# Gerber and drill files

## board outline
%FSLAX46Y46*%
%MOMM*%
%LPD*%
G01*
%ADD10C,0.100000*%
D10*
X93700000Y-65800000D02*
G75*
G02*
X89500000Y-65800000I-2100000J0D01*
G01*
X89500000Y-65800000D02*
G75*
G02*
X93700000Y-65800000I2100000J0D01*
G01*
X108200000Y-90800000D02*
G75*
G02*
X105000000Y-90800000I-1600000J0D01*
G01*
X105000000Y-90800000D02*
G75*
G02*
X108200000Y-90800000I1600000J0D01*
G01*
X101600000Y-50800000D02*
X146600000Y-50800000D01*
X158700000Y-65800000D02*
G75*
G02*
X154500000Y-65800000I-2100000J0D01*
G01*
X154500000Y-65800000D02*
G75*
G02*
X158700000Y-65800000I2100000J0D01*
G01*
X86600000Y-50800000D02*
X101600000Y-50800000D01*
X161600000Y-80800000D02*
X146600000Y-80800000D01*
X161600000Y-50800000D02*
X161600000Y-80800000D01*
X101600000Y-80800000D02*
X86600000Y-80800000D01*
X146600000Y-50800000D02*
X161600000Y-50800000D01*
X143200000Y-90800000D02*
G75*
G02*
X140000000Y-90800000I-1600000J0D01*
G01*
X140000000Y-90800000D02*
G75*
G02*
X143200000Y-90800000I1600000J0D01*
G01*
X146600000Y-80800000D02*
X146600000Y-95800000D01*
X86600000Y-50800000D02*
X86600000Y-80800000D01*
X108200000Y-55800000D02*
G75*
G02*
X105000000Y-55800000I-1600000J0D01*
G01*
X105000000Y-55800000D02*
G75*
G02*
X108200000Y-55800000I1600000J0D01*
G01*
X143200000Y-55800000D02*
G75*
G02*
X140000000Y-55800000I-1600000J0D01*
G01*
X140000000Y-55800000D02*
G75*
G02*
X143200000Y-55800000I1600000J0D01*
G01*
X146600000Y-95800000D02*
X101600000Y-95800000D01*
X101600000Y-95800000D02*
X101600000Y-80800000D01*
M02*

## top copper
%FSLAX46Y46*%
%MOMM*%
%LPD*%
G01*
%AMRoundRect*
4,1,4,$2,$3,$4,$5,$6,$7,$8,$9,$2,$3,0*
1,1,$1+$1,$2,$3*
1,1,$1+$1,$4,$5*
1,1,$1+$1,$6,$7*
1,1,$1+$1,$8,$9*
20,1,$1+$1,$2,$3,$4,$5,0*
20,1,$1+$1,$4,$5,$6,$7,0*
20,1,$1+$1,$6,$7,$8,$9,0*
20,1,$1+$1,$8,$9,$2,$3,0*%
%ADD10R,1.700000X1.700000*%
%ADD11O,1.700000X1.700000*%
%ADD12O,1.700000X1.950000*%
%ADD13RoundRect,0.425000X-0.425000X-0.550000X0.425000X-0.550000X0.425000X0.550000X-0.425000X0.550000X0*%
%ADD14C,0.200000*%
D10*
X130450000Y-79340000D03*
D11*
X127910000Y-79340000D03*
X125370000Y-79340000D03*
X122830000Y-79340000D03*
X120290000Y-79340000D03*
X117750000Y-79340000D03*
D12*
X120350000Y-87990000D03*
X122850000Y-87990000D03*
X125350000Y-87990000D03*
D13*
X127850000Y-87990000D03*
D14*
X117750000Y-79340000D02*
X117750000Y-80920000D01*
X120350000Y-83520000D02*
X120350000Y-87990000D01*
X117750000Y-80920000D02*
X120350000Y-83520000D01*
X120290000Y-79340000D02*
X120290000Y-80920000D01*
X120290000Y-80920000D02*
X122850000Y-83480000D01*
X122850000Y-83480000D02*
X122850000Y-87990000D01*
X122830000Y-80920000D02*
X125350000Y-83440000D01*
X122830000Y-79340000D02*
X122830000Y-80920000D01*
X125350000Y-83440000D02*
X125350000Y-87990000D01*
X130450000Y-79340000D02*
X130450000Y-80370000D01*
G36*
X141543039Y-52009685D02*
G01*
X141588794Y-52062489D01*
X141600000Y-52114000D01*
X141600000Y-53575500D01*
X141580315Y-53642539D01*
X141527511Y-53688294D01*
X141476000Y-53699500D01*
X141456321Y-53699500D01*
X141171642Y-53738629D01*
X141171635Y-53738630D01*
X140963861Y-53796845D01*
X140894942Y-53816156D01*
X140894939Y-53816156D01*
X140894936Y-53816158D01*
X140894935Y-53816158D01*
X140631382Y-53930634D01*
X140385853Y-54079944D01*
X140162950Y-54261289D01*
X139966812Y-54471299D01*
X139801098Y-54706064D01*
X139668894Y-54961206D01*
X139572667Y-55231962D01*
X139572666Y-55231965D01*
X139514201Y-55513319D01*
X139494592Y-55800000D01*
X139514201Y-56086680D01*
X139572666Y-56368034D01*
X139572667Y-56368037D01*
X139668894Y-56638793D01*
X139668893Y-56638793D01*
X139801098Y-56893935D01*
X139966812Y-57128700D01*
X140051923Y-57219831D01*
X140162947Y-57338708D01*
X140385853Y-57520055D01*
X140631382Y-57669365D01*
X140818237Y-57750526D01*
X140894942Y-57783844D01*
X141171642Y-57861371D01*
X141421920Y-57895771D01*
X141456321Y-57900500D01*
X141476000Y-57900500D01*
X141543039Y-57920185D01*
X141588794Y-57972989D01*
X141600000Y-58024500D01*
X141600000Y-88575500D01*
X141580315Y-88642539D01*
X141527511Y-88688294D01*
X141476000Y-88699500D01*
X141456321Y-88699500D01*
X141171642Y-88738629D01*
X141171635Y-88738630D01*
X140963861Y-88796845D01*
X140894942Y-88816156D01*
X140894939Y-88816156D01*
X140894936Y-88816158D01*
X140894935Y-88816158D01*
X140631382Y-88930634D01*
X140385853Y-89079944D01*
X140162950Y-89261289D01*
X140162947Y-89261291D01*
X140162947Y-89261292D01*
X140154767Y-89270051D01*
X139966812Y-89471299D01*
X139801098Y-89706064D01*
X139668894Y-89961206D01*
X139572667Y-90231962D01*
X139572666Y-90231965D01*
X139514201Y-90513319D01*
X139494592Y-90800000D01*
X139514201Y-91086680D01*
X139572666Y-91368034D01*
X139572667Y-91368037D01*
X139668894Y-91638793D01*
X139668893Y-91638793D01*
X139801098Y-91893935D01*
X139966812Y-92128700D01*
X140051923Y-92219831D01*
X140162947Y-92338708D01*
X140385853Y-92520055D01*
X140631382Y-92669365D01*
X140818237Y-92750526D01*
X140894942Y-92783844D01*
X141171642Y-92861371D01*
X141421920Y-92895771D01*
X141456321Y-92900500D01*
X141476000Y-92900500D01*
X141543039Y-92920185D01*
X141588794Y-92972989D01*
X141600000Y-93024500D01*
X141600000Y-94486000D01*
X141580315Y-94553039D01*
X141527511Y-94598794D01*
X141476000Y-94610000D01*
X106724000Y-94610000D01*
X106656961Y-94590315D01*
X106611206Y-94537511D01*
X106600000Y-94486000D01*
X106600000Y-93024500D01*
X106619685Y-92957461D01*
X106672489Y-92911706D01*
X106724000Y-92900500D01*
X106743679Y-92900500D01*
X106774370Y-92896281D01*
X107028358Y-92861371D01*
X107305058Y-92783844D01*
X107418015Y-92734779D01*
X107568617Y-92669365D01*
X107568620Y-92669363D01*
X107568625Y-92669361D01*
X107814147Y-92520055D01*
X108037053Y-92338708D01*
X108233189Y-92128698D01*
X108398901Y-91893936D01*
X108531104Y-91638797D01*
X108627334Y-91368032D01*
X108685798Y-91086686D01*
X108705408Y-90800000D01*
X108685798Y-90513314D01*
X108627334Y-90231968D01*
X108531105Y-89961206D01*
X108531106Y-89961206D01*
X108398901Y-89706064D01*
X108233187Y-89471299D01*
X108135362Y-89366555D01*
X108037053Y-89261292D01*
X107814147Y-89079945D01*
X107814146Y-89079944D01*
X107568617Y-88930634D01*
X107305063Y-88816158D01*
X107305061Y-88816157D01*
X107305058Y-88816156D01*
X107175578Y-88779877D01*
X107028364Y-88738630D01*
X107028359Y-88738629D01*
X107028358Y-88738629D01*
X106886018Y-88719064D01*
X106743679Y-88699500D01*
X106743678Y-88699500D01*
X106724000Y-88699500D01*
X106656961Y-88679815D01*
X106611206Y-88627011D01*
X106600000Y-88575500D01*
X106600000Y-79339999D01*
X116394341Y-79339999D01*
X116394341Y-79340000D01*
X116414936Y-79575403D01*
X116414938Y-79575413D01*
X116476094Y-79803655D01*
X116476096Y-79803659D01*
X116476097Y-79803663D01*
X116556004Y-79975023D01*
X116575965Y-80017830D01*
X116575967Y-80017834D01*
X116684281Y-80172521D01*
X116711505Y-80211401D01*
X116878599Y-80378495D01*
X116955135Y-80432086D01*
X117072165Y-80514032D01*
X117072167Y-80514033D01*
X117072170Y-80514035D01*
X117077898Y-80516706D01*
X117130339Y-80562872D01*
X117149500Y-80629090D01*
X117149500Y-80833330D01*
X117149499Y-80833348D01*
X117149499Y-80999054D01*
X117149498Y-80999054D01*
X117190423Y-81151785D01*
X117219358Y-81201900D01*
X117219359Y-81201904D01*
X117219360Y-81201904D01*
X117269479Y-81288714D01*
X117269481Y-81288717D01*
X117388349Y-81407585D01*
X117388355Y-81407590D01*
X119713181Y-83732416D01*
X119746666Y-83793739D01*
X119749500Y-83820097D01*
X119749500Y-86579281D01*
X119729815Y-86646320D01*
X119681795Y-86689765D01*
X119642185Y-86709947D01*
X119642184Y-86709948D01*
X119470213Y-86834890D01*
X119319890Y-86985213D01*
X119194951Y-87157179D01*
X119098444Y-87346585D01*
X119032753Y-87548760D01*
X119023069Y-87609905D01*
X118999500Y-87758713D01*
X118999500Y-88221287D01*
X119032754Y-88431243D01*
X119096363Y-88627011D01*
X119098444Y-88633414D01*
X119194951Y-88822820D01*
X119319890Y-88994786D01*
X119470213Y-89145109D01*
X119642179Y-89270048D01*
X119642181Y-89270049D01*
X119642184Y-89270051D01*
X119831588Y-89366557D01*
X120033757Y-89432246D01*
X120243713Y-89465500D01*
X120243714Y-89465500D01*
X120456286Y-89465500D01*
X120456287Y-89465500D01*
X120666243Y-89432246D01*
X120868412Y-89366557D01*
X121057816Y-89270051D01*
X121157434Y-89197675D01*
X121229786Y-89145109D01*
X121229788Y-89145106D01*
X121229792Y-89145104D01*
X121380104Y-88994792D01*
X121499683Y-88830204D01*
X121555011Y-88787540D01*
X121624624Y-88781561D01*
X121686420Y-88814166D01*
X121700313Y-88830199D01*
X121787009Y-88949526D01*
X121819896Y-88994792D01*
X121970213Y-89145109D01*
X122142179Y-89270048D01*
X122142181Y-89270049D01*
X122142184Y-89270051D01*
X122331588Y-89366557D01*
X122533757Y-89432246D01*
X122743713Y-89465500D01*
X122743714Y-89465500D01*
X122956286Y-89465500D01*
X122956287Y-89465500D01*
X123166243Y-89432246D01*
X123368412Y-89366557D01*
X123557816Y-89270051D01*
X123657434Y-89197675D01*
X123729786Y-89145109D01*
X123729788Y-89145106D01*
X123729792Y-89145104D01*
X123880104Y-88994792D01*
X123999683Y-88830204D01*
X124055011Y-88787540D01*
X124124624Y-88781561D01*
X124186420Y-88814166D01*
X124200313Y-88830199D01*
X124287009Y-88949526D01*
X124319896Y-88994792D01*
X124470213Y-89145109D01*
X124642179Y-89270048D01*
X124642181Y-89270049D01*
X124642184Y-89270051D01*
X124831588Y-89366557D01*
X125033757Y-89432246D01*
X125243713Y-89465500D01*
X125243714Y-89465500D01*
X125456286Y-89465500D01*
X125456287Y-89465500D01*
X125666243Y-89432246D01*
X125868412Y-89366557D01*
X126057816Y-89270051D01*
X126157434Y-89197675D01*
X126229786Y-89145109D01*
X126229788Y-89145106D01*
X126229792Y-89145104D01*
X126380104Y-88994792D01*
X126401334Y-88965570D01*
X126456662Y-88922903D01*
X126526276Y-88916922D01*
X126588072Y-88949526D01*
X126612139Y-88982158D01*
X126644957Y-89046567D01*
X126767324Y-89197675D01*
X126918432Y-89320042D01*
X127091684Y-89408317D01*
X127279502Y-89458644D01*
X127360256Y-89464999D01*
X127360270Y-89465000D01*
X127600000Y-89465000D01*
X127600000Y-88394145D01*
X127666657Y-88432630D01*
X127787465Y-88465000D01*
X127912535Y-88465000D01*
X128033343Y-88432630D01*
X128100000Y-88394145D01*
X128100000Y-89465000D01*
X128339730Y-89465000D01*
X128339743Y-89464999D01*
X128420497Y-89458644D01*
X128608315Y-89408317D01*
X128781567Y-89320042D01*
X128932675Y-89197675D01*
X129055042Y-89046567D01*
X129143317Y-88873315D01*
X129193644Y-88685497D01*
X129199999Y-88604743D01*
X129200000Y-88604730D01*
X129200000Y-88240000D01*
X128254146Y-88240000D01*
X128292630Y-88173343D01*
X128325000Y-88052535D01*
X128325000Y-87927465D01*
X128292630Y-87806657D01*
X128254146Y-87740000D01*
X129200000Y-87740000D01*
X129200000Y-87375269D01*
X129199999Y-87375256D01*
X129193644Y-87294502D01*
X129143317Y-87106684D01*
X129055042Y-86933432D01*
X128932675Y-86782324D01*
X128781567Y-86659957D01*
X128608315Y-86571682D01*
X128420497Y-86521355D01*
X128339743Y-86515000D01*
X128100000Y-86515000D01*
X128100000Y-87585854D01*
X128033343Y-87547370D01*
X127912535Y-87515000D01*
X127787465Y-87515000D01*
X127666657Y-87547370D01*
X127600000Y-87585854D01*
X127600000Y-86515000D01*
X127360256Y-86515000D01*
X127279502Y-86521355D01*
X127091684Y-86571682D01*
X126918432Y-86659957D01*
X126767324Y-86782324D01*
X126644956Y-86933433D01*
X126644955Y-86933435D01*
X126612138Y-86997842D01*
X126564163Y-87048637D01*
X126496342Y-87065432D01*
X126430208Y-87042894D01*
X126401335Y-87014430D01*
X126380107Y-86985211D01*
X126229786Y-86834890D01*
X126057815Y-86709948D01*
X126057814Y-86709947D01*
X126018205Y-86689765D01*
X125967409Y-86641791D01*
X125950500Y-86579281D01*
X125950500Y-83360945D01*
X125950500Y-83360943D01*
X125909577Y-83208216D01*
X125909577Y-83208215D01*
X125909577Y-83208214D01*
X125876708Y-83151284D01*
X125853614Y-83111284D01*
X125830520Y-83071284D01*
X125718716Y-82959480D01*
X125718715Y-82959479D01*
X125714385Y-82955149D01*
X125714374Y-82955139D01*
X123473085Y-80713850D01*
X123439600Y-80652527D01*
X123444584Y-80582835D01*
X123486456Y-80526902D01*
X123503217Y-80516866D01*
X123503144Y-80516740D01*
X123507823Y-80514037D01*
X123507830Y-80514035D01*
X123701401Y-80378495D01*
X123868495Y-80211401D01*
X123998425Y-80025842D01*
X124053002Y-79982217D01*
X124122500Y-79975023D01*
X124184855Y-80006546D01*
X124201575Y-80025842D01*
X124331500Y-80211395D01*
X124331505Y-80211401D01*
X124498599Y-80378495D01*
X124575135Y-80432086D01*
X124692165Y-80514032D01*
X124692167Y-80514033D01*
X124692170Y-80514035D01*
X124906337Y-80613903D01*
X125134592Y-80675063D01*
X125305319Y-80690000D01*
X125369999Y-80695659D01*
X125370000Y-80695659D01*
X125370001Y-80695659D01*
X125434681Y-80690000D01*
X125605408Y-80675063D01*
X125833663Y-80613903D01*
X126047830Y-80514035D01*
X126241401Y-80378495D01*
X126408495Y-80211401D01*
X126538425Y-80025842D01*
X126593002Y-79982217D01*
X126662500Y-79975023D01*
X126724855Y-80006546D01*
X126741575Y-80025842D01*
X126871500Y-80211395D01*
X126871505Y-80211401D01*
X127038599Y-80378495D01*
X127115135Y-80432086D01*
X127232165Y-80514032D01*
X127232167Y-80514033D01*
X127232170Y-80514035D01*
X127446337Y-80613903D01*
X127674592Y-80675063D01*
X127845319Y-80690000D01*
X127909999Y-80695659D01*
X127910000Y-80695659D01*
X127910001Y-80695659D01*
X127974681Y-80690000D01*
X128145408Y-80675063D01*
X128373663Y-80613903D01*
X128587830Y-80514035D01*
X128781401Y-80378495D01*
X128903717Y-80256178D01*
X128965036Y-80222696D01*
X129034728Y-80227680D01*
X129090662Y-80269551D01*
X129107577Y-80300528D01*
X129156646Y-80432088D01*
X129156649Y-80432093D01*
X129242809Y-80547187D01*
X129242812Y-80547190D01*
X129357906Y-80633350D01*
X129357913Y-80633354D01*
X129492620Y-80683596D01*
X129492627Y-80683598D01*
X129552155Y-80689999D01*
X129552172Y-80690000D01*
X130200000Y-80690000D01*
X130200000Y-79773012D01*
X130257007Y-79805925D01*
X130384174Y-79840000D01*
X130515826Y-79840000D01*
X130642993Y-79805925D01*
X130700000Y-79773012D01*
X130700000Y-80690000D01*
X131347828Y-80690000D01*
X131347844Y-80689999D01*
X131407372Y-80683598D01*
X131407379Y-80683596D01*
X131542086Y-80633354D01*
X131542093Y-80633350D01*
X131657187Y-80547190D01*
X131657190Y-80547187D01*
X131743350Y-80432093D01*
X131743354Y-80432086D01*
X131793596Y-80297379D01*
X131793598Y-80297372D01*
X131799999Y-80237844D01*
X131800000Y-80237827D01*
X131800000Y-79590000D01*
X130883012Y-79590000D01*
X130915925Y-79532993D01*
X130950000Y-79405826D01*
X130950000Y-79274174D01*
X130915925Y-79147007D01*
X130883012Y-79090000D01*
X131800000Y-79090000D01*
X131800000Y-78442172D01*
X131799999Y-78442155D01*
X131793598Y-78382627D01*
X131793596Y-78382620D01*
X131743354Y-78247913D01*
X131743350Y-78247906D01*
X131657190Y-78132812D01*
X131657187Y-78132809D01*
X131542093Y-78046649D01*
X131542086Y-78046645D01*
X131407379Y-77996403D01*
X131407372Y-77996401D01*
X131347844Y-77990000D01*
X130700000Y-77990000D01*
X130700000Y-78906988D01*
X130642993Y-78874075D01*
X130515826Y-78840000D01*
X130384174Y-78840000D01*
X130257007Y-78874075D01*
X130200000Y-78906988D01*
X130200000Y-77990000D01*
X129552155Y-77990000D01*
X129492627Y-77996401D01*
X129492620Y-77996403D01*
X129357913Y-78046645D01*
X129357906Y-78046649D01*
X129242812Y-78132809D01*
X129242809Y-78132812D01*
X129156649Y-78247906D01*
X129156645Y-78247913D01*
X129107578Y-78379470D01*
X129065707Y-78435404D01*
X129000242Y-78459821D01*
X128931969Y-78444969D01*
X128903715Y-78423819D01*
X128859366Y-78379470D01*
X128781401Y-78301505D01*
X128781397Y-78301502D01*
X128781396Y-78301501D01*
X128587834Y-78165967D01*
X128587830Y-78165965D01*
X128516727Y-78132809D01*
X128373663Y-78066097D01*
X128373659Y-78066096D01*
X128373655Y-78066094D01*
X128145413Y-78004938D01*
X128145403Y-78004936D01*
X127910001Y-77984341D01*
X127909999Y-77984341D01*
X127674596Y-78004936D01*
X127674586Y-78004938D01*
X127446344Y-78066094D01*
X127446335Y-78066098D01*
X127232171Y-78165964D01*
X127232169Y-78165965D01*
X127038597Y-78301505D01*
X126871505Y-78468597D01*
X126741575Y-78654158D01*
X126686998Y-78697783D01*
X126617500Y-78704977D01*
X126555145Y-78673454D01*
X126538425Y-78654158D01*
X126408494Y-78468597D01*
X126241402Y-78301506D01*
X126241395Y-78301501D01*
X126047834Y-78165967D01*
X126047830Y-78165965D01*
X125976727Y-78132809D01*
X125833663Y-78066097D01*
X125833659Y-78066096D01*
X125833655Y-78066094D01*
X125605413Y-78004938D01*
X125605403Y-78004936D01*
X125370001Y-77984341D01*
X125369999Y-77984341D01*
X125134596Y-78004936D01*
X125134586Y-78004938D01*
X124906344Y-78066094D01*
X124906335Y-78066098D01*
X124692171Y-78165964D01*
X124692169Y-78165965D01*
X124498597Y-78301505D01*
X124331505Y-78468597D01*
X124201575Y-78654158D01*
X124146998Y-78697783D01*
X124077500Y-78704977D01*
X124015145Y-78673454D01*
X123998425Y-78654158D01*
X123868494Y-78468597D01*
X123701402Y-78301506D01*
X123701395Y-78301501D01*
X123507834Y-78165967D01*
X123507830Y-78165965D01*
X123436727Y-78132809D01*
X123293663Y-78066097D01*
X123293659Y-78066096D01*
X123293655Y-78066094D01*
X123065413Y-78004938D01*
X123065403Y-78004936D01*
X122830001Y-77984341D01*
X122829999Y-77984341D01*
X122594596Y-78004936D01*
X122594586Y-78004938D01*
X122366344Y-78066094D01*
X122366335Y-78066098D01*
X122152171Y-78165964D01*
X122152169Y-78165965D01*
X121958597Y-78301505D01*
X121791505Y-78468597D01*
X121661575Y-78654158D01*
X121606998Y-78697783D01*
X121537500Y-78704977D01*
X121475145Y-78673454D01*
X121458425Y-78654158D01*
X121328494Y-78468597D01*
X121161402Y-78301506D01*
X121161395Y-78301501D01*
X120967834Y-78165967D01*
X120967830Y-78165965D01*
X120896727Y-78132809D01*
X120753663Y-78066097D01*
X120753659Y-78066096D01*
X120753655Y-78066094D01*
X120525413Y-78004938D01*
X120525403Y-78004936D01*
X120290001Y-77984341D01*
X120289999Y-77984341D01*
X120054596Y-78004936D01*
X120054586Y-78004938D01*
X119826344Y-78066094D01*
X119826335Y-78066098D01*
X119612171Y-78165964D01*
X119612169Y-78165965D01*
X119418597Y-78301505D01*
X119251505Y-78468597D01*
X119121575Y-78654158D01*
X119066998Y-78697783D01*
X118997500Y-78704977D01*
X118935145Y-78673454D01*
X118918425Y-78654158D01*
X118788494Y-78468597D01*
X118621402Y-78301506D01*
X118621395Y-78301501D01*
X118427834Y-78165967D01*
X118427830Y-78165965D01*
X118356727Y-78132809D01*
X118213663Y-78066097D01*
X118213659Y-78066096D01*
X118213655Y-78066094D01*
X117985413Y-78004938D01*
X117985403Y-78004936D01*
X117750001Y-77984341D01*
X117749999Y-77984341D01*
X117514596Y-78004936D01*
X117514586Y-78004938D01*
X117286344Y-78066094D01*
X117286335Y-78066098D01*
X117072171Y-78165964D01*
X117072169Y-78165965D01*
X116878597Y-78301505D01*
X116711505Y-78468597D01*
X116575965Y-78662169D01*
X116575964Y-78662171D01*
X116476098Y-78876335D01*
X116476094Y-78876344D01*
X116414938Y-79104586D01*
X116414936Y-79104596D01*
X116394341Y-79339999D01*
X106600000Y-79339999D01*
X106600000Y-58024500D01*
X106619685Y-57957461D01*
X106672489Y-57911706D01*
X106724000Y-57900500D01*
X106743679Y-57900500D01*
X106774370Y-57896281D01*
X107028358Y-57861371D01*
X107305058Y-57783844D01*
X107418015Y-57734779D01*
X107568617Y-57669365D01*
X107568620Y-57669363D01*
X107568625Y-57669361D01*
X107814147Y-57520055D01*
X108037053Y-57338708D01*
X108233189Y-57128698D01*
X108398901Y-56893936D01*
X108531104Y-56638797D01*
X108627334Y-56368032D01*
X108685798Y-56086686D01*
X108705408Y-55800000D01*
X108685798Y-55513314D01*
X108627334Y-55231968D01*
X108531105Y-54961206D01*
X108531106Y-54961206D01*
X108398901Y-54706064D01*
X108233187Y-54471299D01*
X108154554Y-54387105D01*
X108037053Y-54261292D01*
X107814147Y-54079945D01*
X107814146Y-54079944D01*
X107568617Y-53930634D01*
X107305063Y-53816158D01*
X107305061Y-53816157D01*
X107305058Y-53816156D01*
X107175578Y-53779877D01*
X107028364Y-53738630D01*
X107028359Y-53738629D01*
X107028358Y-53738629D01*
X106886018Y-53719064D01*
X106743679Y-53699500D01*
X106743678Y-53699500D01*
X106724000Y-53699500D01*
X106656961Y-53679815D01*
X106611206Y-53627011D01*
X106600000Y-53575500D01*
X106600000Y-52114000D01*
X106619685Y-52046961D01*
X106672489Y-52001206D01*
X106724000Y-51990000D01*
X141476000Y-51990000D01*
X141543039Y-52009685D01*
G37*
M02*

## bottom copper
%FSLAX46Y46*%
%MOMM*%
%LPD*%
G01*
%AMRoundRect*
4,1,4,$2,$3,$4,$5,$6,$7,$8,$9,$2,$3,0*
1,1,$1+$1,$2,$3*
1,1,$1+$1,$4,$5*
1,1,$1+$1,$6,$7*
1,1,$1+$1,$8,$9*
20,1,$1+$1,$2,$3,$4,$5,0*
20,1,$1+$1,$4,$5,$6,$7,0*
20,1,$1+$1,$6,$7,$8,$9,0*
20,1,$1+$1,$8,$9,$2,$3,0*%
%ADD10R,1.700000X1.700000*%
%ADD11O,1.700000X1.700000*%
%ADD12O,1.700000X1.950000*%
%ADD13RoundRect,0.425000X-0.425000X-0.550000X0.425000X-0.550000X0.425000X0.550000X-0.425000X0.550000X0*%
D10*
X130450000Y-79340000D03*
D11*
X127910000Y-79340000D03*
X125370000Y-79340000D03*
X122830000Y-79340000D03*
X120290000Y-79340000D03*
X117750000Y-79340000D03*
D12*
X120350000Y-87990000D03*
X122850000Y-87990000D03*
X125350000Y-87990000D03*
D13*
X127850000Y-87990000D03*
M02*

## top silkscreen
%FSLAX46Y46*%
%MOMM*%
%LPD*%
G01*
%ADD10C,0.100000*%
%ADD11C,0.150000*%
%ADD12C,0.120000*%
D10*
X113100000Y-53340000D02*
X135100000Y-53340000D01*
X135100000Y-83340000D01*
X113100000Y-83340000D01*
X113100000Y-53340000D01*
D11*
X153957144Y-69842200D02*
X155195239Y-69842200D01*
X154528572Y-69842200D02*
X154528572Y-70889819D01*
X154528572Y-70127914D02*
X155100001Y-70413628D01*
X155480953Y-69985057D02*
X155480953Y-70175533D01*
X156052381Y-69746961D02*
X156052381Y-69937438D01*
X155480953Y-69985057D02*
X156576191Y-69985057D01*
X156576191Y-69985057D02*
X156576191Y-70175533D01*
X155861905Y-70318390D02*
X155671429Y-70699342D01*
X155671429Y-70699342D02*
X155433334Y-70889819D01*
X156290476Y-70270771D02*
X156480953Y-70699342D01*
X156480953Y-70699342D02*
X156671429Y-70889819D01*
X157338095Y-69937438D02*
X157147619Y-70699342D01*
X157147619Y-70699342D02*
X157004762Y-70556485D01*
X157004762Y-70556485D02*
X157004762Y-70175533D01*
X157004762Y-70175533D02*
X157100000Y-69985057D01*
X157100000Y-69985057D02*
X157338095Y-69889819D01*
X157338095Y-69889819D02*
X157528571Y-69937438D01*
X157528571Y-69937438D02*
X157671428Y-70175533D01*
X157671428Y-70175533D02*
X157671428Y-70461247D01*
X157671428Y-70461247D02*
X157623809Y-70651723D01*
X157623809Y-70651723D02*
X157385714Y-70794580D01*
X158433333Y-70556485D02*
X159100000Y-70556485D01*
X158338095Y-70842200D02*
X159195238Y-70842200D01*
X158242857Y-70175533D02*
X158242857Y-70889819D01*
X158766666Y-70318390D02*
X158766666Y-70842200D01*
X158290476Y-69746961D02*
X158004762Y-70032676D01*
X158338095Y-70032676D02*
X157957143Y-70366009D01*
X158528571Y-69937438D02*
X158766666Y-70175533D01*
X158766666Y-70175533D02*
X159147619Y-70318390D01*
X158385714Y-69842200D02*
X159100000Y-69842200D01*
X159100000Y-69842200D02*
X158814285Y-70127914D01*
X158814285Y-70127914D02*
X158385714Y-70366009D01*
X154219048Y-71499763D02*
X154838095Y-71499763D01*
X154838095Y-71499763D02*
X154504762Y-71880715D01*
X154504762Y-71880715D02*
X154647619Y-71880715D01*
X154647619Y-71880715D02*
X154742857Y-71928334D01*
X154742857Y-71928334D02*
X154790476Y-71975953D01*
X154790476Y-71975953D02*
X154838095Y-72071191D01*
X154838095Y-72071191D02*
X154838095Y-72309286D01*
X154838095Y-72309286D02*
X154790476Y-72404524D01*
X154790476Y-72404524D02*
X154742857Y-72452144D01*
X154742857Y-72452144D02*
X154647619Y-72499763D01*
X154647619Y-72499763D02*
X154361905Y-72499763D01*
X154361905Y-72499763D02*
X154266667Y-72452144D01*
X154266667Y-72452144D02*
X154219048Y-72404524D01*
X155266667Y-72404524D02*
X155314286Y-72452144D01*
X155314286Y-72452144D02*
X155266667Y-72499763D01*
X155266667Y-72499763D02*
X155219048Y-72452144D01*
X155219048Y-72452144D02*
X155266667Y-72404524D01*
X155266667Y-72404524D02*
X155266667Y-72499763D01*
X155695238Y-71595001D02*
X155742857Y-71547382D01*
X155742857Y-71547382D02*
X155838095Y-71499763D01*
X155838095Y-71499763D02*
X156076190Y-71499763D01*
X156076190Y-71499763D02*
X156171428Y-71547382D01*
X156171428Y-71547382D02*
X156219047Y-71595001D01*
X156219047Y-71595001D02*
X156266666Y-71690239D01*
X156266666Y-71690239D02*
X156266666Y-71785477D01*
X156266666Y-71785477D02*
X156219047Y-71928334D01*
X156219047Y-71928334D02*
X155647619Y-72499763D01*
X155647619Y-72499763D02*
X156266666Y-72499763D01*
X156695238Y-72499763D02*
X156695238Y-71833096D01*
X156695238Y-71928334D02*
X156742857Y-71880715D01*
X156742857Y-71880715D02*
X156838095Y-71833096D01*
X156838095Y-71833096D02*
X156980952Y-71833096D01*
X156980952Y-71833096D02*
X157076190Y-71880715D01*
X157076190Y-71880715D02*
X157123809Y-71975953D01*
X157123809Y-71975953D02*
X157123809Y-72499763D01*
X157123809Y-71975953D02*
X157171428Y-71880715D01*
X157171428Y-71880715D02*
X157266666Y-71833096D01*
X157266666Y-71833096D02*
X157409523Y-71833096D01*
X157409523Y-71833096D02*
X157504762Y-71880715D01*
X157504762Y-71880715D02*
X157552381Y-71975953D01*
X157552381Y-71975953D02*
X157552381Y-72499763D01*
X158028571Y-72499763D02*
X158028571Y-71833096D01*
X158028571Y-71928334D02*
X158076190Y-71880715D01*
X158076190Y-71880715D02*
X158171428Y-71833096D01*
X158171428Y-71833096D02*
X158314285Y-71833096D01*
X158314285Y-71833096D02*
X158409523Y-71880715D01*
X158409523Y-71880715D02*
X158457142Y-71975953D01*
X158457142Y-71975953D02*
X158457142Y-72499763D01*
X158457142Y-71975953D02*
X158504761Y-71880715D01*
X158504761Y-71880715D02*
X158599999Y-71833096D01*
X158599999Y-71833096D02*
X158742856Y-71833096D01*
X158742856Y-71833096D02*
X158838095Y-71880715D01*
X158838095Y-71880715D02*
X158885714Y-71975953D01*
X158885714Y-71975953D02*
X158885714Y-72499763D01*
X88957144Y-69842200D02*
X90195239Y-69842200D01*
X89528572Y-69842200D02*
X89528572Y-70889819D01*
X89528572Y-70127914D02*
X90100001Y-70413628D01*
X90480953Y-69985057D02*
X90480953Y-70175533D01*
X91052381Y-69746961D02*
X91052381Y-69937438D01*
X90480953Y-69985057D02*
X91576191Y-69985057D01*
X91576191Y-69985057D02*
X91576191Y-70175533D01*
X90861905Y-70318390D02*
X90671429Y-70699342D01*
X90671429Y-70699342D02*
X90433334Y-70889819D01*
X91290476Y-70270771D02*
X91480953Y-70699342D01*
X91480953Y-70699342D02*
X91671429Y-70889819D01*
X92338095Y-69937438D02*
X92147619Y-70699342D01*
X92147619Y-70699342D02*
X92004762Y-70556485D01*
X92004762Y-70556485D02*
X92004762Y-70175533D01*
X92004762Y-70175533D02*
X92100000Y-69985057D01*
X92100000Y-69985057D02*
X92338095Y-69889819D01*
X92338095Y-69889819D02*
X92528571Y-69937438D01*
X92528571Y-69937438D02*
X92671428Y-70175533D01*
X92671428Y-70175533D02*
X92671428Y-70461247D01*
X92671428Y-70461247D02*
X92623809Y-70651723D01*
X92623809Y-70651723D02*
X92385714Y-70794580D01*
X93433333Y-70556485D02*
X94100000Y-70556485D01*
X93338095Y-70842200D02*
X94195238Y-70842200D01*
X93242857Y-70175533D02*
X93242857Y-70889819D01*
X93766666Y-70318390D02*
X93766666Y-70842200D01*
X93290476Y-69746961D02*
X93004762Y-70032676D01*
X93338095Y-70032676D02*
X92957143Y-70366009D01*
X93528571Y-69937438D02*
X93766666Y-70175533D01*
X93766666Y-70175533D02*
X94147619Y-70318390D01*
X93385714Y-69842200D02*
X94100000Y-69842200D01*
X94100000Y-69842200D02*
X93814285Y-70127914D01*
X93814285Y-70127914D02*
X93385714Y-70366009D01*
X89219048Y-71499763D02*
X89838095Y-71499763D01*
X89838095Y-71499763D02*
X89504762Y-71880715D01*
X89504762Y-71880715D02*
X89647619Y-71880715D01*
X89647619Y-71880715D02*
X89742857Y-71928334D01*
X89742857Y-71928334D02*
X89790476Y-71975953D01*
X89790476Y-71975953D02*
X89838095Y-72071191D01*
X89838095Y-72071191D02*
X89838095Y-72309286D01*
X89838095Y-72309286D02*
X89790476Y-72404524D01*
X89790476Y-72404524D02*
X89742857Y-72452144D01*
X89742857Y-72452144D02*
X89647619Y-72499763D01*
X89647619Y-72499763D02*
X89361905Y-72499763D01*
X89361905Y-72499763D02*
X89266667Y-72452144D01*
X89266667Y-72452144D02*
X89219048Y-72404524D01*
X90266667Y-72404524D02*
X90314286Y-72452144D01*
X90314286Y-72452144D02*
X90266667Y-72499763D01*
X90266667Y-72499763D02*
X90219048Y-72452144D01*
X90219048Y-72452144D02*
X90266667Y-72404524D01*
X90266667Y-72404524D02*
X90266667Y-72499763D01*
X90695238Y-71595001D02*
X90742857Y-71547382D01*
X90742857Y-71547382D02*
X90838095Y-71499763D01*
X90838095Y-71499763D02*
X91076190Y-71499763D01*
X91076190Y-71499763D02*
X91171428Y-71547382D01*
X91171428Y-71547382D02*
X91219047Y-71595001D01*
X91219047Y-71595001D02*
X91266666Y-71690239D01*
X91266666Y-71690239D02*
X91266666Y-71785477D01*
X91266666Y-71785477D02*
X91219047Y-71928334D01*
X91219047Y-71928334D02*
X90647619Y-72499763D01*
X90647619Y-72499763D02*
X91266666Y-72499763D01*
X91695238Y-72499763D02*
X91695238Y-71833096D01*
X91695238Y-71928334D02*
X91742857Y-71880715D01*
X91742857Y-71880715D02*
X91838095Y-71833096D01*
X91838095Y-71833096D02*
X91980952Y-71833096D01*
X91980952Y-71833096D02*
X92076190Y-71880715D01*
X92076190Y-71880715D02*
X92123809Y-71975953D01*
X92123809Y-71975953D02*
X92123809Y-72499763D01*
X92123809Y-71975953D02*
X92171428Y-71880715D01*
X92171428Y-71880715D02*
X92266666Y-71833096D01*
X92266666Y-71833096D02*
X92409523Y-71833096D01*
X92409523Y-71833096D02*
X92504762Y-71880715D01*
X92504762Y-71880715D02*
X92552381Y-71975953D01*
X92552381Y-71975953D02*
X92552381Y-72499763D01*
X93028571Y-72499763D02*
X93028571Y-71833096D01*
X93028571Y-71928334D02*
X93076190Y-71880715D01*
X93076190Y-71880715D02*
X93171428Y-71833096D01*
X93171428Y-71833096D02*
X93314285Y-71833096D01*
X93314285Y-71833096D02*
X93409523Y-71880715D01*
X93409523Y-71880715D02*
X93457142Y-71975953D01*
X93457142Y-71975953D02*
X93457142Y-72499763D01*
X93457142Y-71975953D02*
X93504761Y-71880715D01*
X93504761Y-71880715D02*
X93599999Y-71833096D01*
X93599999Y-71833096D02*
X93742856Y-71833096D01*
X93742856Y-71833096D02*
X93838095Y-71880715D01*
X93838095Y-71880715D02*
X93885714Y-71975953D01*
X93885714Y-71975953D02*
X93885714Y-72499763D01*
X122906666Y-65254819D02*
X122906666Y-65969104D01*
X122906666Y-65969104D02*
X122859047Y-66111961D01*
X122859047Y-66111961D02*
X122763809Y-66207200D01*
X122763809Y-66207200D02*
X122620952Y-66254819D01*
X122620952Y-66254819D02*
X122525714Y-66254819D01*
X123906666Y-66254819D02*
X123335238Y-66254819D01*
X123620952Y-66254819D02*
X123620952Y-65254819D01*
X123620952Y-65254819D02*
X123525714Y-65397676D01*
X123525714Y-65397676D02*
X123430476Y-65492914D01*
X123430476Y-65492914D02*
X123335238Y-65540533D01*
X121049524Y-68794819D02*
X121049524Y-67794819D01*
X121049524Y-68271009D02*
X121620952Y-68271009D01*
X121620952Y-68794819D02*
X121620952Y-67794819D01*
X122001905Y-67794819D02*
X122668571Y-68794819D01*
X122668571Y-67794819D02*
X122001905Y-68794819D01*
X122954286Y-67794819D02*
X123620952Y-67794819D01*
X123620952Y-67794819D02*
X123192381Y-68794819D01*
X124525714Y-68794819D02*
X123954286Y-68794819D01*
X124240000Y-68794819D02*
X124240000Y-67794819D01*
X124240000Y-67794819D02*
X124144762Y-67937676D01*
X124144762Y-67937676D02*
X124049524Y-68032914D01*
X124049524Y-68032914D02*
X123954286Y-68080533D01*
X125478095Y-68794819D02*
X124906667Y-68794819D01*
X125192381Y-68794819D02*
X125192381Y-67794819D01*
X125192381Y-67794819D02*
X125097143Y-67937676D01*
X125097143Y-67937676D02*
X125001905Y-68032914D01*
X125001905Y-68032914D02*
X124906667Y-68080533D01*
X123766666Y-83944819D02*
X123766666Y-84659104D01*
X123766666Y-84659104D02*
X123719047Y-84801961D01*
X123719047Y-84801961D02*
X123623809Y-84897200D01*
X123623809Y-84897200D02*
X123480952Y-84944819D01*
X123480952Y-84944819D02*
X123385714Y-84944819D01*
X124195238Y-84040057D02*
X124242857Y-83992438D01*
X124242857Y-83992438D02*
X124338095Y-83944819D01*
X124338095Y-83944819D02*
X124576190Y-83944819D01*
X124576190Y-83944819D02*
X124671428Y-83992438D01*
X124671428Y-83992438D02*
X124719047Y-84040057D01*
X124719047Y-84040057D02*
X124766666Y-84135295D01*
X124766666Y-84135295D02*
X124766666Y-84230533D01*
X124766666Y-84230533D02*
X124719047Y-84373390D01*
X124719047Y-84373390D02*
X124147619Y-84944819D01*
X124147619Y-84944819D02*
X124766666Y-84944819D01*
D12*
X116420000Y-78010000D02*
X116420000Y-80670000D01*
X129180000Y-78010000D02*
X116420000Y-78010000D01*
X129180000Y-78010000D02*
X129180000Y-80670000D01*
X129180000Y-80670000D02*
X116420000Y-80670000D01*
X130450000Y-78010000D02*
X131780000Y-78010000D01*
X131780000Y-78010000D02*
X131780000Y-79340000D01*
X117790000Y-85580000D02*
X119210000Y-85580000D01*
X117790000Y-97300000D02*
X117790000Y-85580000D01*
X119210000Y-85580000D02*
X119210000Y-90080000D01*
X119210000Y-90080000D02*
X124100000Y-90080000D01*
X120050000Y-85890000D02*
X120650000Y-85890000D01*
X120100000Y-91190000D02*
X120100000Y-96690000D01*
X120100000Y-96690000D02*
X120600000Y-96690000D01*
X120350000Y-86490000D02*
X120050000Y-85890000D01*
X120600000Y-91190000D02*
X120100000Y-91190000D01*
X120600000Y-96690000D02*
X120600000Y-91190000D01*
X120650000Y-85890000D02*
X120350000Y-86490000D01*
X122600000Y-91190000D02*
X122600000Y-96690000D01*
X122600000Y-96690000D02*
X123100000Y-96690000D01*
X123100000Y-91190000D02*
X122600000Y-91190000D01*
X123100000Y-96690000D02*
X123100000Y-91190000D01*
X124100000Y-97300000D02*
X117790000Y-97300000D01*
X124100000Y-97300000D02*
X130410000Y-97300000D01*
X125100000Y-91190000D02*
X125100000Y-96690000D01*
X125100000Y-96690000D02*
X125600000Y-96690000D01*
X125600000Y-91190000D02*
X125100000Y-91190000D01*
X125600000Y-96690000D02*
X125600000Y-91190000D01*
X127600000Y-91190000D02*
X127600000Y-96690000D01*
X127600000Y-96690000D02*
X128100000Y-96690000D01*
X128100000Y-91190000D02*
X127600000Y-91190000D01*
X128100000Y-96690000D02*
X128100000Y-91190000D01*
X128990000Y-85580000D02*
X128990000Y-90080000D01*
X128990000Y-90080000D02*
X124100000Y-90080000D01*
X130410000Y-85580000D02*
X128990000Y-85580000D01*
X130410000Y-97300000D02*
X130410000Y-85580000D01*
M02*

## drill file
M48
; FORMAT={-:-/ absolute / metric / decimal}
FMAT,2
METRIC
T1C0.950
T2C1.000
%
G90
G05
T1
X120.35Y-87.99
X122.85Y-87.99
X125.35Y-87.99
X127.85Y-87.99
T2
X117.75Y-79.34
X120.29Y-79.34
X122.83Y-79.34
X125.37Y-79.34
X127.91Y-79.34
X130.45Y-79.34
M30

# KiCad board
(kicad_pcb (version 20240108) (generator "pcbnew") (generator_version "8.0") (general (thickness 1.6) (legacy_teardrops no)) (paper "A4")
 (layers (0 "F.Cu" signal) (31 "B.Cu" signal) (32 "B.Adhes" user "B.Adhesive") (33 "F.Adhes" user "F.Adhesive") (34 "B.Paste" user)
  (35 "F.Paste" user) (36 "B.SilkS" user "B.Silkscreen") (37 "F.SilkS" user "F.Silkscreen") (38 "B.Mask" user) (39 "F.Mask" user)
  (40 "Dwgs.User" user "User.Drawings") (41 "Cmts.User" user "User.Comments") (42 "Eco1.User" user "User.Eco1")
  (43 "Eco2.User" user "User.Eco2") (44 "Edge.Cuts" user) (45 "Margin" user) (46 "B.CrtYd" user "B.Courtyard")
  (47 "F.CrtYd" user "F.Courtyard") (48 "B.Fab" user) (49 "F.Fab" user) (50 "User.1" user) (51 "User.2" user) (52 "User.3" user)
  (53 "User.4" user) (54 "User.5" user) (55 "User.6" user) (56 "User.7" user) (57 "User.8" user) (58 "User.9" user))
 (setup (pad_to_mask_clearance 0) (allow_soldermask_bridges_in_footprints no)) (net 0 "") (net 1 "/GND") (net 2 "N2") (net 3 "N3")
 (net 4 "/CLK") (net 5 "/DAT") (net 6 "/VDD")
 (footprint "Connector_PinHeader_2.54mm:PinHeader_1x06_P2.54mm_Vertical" (layer "F.Cu") (at 130.45 79.34 -90)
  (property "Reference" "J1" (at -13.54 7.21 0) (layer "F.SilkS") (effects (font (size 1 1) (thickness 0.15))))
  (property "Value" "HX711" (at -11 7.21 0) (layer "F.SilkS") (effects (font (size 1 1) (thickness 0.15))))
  (fp_line (start -1.33 14.03) (end 1.33 14.03) (stroke (width 0.12) (type solid)) (layer "F.SilkS"))
  (fp_line (start -1.33 1.27) (end -1.33 14.03) (stroke (width 0.12) (type solid)) (layer "F.SilkS"))
  (fp_line (start -1.33 1.27) (end 1.33 1.27) (stroke (width 0.12) (type solid)) (layer "F.SilkS"))
  (fp_line (start 1.33 1.27) (end 1.33 14.03) (stroke (width 0.12) (type solid)) (layer "F.SilkS"))
  (fp_line (start -1.33 0) (end -1.33 -1.33) (stroke (width 0.12) (type solid)) (layer "F.SilkS"))
  (fp_line (start -1.33 -1.33) (end 0 -1.33) (stroke (width 0.12) (type solid)) (layer "F.SilkS"))
  (pad "1" thru_hole rect (at 0 0 270) (size 1.7 1.7) (drill 1) (layers "*.Cu" "*.Mask") (remove_unused_layers no) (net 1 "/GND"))
  (pad "2" thru_hole oval (at 0 2.54 270) (size 1.7 1.7) (drill 1) (layers "*.Cu" "*.Mask") (remove_unused_layers no) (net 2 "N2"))
  (pad "3" thru_hole oval (at 0 5.08 270) (size 1.7 1.7) (drill 1) (layers "*.Cu" "*.Mask") (remove_unused_layers no) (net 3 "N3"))
  (pad "4" thru_hole oval (at 0 7.62 270) (size 1.7 1.7) (drill 1) (layers "*.Cu" "*.Mask") (remove_unused_layers no) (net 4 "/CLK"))
  (pad "5" thru_hole oval (at 0 10.16 270) (size 1.7 1.7) (drill 1) (layers "*.Cu" "*.Mask") (remove_unused_layers no) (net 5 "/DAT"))
  (pad "6" thru_hole oval (at 0 12.7 270) (size 1.7 1.7) (drill 1) (layers "*.Cu" "*.Mask") (remove_unused_layers no) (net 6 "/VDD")))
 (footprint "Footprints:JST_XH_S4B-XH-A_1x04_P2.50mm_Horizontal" (layer "F.Cu") (at 120.35 87.99)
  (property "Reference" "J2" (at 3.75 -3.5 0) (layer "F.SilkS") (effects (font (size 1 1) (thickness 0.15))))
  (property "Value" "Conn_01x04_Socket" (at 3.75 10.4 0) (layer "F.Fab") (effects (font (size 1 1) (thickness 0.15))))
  (fp_line (start -2.56 -2.41) (end -1.14 -2.41) (stroke (width 0.12) (type solid)) (layer "F.SilkS"))
  (fp_line (start -2.56 9.31) (end -2.56 -2.41) (stroke (width 0.12) (type solid)) (layer "F.SilkS"))
  (fp_line (start -1.14 -2.41) (end -1.14 2.09) (stroke (width 0.12) (type solid)) (layer "F.SilkS"))
  (fp_line (start -1.14 2.09) (end 3.75 2.09) (stroke (width 0.12) (type solid)) (layer "F.SilkS"))
  (fp_line (start -0.3 -2.1) (end 0.3 -2.1) (stroke (width 0.12) (type solid)) (layer "F.SilkS"))
  (fp_line (start -0.25 3.2) (end -0.25 8.7) (stroke (width 0.12) (type solid)) (layer "F.SilkS"))
  (fp_line (start -0.25 8.7) (end 0.25 8.7) (stroke (width 0.12) (type solid)) (layer "F.SilkS"))
  (fp_line (start 0 -1.5) (end -0.3 -2.1) (stroke (width 0.12) (type solid)) (layer "F.SilkS"))
  (fp_line (start 0.25 3.2) (end -0.25 3.2) (stroke (width 0.12) (type solid)) (layer "F.SilkS"))
  (fp_line (start 0.25 8.7) (end 0.25 3.2) (stroke (width 0.12) (type solid)) (layer "F.SilkS"))
  (fp_line (start 0.3 -2.1) (end 0 -1.5) (stroke (width 0.12) (type solid)) (layer "F.SilkS"))
  (fp_line (start 2.25 3.2) (end 2.25 8.7) (stroke (width 0.12) (type solid)) (layer "F.SilkS"))
  (fp_line (start 2.25 8.7) (end 2.75 8.7) (stroke (width 0.12) (type solid)) (layer "F.SilkS"))
  (fp_line (start 2.75 3.2) (end 2.25 3.2) (stroke (width 0.12) (type solid)) (layer "F.SilkS"))
  (fp_line (start 2.75 8.7) (end 2.75 3.2) (stroke (width 0.12) (type solid)) (layer "F.SilkS"))
  (fp_line (start 3.75 9.31) (end -2.56 9.31) (stroke (width 0.12) (type solid)) (layer "F.SilkS"))
  (fp_line (start 3.75 9.31) (end 10.06 9.31) (stroke (width 0.12) (type solid)) (layer "F.SilkS"))
  (fp_line (start 4.75 3.2) (end 4.75 8.7) (stroke (width 0.12) (type solid)) (layer "F.SilkS"))
  (fp_line (start 4.75 8.7) (end 5.25 8.7) (stroke (width 0.12) (type solid)) (layer "F.SilkS"))
  (fp_line (start 5.25 3.2) (end 4.75 3.2) (stroke (width 0.12) (type solid)) (layer "F.SilkS"))
  (fp_line (start 5.25 8.7) (end 5.25 3.2) (stroke (width 0.12) (type solid)) (layer "F.SilkS"))
  (fp_line (start 7.25 3.2) (end 7.25 8.7) (stroke (width 0.12) (type solid)) (layer "F.SilkS"))
  (fp_line (start 7.25 8.7) (end 7.75 8.7) (stroke (width 0.12) (type solid)) (layer "F.SilkS"))
  (fp_line (start 7.75 3.2) (end 7.25 3.2) (stroke (width 0.12) (type solid)) (layer "F.SilkS"))
  (fp_line (start 7.75 8.7) (end 7.75 3.2) (stroke (width 0.12) (type solid)) (layer "F.SilkS"))
  (fp_line (start 8.64 -2.41) (end 8.64 2.09) (stroke (width 0.12) (type solid)) (layer "F.SilkS"))
  (fp_line (start 8.64 2.09) (end 3.75 2.09) (stroke (width 0.12) (type solid)) (layer "F.SilkS"))
  (fp_line (start 10.06 -2.41) (end 8.64 -2.41) (stroke (width 0.12) (type solid)) (layer "F.SilkS"))
  (fp_line (start 10.06 9.31) (end 10.06 -2.41) (stroke (width 0.12) (type solid)) (layer "F.SilkS"))
  (pad "1" thru_hole oval (at 0 0) (size 1.7 1.95) (drill 0.95) (layers "*.Cu" "*.Mask") (remove_unused_layers no) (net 6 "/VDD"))
  (pad "2" thru_hole oval (at 2.5 0) (size 1.7 1.95) (drill 0.95) (layers "*.Cu" "*.Mask") (remove_unused_layers no) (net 5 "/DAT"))
  (pad "3" thru_hole oval (at 5 0) (size 1.7 1.95) (drill 0.95) (layers "*.Cu" "*.Mask") (remove_unused_layers no) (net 4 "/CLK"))
  (pad "4" thru_hole roundrect (at 7.5 0) (size 1.7 1.95) (drill 0.95) (layers "*.Cu" "*.Mask") (remove_unused_layers no)
   (roundrect_rratio 0.25) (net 1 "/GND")))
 (gr_rect (start 113.1 53.34) (end 135.1 83.34) (stroke (width 0.1) (type default)) (fill none) (layer "F.SilkS"))
 (gr_circle (center 91.6 65.8) (end 93.7 65.8) (stroke (width 0.1) (type default)) (fill none) (layer "Edge.Cuts"))
 (gr_circle (center 106.6 90.8) (end 108.2 90.8) (stroke (width 0.1) (type default)) (fill none) (layer "Edge.Cuts"))
 (gr_line (start 101.6 50.8) (end 146.6 50.8) (stroke (width 0.1) (type default)) (layer "Edge.Cuts"))
 (gr_circle (center 156.6 65.8) (end 158.7 65.8) (stroke (width 0.1) (type default)) (fill none) (layer "Edge.Cuts"))
 (gr_line (start 86.6 50.8) (end 101.6 50.8) (stroke (width 0.1) (type default)) (layer "Edge.Cuts"))
 (gr_line (start 161.6 80.8) (end 146.6 80.8) (stroke (width 0.1) (type default)) (layer "Edge.Cuts"))
 (gr_line (start 161.6 50.8) (end 161.6 80.8) (stroke (width 0.1) (type default)) (layer "Edge.Cuts"))
 (gr_line (start 101.6 80.8) (end 86.6 80.8) (stroke (width 0.1) (type default)) (layer "Edge.Cuts"))
 (gr_line (start 146.6 50.8) (end 161.6 50.8) (stroke (width 0.1) (type default)) (layer "Edge.Cuts"))
 (gr_circle (center 141.6 90.8) (end 143.2 90.8) (stroke (width 0.1) (type default)) (fill none) (layer "Edge.Cuts"))
 (gr_line (start 146.6 80.8) (end 146.6 95.8) (stroke (width 0.1) (type default)) (layer "Edge.Cuts"))
 (gr_line (start 86.6 50.8) (end 86.6 80.8) (stroke (width 0.1) (type default)) (layer "Edge.Cuts"))
 (gr_circle (center 106.6 55.8) (end 108.2 55.8) (stroke (width 0.1) (type default)) (fill none) (layer "Edge.Cuts"))
 (gr_circle (center 141.6 55.8) (end 143.2 55.8) (stroke (width 0.1) (type default)) (fill none) (layer "Edge.Cuts"))
 (gr_line (start 146.6 95.8) (end 101.6 95.8) (stroke (width 0.1) (type default)) (layer "Edge.Cuts"))
 (gr_line (start 101.6 95.8) (end 101.6 80.8) (stroke (width 0.1) (type default)) (layer "Edge.Cuts"))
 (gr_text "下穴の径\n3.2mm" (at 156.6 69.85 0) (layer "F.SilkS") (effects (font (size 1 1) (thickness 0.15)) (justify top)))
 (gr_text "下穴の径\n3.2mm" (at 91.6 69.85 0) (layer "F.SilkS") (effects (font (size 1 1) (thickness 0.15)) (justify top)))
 (segment (start 117.75 79.34) (end 117.75 80.92) (width 0.2) (layer "F.Cu") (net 6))
 (segment (start 120.35 83.52) (end 120.35 87.99) (width 0.2) (layer "F.Cu") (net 6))
 (segment (start 117.75 80.92) (end 120.35 83.52) (width 0.2) (layer "F.Cu") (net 6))
 (segment (start 120.29 79.34) (end 120.29 80.92) (width 0.2) (layer "F.Cu") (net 5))
 (segment (start 120.29 80.92) (end 122.85 83.48) (width 0.2) (layer "F.Cu") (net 5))
 (segment (start 122.85 83.48) (end 122.85 87.99) (width 0.2) (layer "F.Cu") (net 5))
 (segment (start 122.83 80.92) (end 125.35 83.44) (width 0.2) (layer "F.Cu") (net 4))
 (segment (start 122.83 79.34) (end 122.83 80.92) (width 0.2) (layer "F.Cu") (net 4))
 (segment (start 125.35 83.44) (end 125.35 87.99) (width 0.2) (layer "F.Cu") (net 4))
 (segment (start 130.45 79.34) (end 130.45 80.37) (width 0.2) (layer "F.Cu") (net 1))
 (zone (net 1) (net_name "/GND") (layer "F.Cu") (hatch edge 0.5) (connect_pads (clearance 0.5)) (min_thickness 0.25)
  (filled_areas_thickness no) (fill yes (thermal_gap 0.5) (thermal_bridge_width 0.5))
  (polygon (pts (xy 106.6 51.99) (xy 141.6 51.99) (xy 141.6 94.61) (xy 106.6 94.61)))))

